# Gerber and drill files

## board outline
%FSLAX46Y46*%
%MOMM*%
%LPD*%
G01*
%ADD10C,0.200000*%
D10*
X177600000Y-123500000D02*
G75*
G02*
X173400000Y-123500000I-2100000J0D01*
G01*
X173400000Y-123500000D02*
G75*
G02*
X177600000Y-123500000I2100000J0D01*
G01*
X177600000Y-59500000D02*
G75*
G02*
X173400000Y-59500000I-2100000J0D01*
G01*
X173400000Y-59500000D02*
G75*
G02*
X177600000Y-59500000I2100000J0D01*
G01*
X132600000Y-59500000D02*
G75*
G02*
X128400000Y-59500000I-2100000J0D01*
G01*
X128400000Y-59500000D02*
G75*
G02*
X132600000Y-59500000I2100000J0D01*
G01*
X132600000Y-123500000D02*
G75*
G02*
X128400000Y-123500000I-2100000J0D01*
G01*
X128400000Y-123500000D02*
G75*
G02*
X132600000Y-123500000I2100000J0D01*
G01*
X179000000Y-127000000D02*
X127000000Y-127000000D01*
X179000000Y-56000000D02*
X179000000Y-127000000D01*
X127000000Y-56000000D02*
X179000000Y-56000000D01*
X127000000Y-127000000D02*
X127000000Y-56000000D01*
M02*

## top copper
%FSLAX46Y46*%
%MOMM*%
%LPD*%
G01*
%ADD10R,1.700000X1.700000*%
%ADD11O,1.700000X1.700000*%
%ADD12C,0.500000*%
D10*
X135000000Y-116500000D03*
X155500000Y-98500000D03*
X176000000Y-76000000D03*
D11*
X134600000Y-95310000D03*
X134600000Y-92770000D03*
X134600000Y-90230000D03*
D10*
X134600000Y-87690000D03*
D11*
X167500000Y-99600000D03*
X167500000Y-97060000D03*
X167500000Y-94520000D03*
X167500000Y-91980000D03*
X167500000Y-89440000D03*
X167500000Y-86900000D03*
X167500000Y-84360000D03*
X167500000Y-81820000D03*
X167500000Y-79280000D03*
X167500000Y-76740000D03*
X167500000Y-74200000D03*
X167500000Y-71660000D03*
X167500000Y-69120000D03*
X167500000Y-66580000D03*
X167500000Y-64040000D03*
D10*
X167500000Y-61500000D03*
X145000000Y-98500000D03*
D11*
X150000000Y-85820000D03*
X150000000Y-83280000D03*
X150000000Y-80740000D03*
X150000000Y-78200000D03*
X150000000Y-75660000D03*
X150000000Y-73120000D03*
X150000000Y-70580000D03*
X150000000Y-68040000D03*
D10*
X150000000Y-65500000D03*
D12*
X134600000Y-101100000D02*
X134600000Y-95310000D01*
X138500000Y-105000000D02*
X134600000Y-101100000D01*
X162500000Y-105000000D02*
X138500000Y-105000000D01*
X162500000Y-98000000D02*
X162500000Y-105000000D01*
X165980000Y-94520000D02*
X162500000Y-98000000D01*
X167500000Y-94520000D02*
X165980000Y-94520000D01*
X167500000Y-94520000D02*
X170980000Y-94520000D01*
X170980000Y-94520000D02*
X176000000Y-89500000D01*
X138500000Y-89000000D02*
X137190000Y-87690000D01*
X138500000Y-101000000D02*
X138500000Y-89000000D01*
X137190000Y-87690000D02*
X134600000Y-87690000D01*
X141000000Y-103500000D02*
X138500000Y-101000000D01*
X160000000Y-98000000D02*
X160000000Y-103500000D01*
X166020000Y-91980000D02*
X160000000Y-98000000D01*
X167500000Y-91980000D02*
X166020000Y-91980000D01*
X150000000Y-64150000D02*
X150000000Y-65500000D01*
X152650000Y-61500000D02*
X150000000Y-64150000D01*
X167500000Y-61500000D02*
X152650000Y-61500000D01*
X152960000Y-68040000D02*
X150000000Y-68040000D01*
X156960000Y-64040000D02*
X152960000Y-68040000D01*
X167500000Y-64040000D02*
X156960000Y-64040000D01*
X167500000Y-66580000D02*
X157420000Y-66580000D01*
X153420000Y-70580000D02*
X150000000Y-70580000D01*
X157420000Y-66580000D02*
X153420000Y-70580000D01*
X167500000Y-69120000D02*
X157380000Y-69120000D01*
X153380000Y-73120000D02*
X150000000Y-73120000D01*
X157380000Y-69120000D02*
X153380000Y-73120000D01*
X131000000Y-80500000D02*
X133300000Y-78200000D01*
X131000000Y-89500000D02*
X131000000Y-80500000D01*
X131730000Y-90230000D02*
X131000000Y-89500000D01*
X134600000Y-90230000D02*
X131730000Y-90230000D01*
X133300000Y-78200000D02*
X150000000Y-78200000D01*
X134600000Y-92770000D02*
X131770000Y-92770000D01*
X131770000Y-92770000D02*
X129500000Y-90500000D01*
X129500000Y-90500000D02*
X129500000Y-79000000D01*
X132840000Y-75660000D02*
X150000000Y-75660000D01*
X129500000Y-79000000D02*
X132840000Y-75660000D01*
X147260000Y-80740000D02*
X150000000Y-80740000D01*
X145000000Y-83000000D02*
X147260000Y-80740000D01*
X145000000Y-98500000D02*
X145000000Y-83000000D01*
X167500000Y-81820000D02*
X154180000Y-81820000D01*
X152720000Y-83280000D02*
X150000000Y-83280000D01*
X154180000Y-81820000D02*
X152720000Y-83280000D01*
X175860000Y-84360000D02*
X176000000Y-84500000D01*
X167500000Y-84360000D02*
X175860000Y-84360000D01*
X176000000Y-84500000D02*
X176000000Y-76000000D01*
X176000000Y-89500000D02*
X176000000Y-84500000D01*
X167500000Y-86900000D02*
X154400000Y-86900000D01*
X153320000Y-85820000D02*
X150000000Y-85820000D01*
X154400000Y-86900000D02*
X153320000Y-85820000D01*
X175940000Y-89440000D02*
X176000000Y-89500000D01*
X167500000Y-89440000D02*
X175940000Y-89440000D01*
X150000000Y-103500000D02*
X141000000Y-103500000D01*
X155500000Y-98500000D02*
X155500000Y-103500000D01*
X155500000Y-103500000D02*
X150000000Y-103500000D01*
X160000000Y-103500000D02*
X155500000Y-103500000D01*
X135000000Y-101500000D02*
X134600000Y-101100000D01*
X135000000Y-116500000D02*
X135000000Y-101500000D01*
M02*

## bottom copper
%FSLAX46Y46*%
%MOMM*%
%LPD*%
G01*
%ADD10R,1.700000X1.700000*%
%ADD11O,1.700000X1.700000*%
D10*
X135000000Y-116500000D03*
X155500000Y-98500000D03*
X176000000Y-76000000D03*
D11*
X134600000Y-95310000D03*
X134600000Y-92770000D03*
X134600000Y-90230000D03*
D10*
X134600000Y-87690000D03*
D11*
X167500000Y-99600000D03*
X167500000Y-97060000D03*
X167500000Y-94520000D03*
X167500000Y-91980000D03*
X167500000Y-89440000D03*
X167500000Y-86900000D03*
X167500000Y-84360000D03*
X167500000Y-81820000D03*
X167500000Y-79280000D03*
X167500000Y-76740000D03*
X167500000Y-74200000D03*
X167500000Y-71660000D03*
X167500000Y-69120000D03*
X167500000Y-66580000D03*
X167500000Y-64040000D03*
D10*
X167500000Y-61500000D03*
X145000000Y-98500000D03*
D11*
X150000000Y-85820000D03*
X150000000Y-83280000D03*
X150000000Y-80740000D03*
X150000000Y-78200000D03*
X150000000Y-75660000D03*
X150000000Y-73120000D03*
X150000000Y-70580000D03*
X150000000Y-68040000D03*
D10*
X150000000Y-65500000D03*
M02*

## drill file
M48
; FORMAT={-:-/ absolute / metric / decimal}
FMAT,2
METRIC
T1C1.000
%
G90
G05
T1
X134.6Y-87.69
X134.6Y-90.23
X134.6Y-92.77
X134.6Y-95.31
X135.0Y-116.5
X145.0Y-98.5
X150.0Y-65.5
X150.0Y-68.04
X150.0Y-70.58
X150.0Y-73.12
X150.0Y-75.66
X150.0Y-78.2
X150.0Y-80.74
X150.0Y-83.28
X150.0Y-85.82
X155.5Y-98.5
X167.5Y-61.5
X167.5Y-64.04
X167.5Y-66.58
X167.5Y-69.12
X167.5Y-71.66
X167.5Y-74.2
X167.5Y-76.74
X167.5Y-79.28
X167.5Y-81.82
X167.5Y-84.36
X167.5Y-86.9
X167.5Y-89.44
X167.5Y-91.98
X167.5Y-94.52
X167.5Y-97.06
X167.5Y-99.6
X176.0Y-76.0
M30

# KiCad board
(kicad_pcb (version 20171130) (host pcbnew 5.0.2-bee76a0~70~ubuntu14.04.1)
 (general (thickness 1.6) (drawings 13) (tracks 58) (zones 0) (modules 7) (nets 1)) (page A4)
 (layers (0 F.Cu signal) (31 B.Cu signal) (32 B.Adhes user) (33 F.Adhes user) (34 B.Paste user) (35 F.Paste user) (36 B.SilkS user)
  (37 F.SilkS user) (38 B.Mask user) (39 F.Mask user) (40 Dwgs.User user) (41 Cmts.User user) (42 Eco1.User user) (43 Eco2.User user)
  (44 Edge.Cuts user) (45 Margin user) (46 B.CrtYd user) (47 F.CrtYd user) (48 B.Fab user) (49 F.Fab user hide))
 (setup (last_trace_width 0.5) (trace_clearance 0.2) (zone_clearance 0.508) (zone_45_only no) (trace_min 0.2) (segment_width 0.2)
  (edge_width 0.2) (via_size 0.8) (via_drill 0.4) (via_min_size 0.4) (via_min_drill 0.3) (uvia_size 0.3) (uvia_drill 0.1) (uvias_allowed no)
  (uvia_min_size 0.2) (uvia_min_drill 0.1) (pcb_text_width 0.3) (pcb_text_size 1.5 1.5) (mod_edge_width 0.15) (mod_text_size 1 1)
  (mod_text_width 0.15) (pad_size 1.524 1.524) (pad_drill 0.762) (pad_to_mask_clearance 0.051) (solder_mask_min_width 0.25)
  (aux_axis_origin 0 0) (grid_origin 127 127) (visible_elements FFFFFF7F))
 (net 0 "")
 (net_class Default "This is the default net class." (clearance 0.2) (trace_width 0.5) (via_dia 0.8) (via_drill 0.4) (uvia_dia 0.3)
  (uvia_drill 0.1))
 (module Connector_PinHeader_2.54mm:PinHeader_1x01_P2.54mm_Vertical (layer F.Cu) (at 135 116.5)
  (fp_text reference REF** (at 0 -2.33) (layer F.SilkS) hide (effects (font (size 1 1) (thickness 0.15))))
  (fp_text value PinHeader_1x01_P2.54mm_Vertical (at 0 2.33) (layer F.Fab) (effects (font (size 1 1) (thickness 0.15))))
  (pad 1 thru_hole rect (at 0 0) (size 1.7 1.7) (drill 1) (layers *.Cu *.Mask)))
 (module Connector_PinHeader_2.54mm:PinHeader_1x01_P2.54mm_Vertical (layer F.Cu) (at 155.5 98.5)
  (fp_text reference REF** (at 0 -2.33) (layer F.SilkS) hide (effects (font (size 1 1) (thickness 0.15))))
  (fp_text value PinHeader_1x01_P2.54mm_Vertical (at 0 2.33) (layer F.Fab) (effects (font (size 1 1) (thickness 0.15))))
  (pad 1 thru_hole rect (at 0 0) (size 1.7 1.7) (drill 1) (layers *.Cu *.Mask)))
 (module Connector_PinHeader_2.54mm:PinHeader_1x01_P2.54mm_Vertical (layer F.Cu) (at 176 76)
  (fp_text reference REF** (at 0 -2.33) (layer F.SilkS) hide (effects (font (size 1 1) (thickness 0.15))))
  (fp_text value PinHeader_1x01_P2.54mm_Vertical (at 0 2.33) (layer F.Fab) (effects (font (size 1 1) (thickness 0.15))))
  (pad 1 thru_hole rect (at 0 0) (size 1.7 1.7) (drill 1) (layers *.Cu *.Mask)))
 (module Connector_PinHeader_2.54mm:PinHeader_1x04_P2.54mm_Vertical (layer F.Cu) (at 134.6 87.69)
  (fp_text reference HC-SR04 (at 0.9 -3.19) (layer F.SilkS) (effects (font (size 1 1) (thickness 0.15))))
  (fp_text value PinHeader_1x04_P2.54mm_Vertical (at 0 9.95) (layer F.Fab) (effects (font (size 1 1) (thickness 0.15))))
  (pad 4 thru_hole oval (at 0 7.62) (size 1.7 1.7) (drill 1) (layers *.Cu *.Mask))
  (pad 3 thru_hole oval (at 0 5.08) (size 1.7 1.7) (drill 1) (layers *.Cu *.Mask))
  (pad 2 thru_hole oval (at 0 2.54) (size 1.7 1.7) (drill 1) (layers *.Cu *.Mask))
  (pad 1 thru_hole rect (at 0 0) (size 1.7 1.7) (drill 1) (layers *.Cu *.Mask)))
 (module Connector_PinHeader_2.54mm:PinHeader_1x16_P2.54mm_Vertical (layer F.Cu) (at 167.5 61.5)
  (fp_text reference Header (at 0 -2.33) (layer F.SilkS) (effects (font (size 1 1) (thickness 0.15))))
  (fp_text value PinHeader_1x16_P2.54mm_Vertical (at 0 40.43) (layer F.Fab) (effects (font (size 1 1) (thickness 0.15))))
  (pad 16 thru_hole oval (at 0 38.1) (size 1.7 1.7) (drill 1) (layers *.Cu *.Mask))
  (pad 15 thru_hole oval (at 0 35.56) (size 1.7 1.7) (drill 1) (layers *.Cu *.Mask))
  (pad 14 thru_hole oval (at 0 33.02) (size 1.7 1.7) (drill 1) (layers *.Cu *.Mask))
  (pad 13 thru_hole oval (at 0 30.48) (size 1.7 1.7) (drill 1) (layers *.Cu *.Mask))
  (pad 12 thru_hole oval (at 0 27.94) (size 1.7 1.7) (drill 1) (layers *.Cu *.Mask))
  (pad 11 thru_hole oval (at 0 25.4) (size 1.7 1.7) (drill 1) (layers *.Cu *.Mask))
  (pad 10 thru_hole oval (at 0 22.86) (size 1.7 1.7) (drill 1) (layers *.Cu *.Mask))
  (pad 9 thru_hole oval (at 0 20.32) (size 1.7 1.7) (drill 1) (layers *.Cu *.Mask))
  (pad 8 thru_hole oval (at 0 17.78) (size 1.7 1.7) (drill 1) (layers *.Cu *.Mask))
  (pad 7 thru_hole oval (at 0 15.24) (size 1.7 1.7) (drill 1) (layers *.Cu *.Mask))
  (pad 6 thru_hole oval (at 0 12.7) (size 1.7 1.7) (drill 1) (layers *.Cu *.Mask))
  (pad 5 thru_hole oval (at 0 10.16) (size 1.7 1.7) (drill 1) (layers *.Cu *.Mask))
  (pad 4 thru_hole oval (at 0 7.62) (size 1.7 1.7) (drill 1) (layers *.Cu *.Mask))
  (pad 3 thru_hole oval (at 0 5.08) (size 1.7 1.7) (drill 1) (layers *.Cu *.Mask))
  (pad 2 thru_hole oval (at 0 2.54) (size 1.7 1.7) (drill 1) (layers *.Cu *.Mask))
  (pad 1 thru_hole rect (at 0 0) (size 1.7 1.7) (drill 1) (layers *.Cu *.Mask)))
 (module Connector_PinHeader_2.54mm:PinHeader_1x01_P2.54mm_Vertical (layer F.Cu) (at 145 98.5)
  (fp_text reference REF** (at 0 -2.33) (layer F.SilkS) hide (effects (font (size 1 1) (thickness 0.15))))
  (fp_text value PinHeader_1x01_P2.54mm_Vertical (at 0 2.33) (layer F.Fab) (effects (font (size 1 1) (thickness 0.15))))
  (pad 1 thru_hole rect (at 0 0) (size 1.7 1.7) (drill 1) (layers *.Cu *.Mask)))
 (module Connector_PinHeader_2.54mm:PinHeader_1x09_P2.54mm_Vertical (layer F.Cu) (at 150 65.5)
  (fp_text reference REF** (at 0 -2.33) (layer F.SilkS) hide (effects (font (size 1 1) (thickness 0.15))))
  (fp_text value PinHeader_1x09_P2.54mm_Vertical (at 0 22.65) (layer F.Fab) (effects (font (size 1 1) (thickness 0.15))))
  (pad 9 thru_hole oval (at 0 20.32) (size 1.7 1.7) (drill 1) (layers *.Cu *.Mask))
  (pad 8 thru_hole oval (at 0 17.78) (size 1.7 1.7) (drill 1) (layers *.Cu *.Mask))
  (pad 7 thru_hole oval (at 0 15.24) (size 1.7 1.7) (drill 1) (layers *.Cu *.Mask))
  (pad 6 thru_hole oval (at 0 12.7) (size 1.7 1.7) (drill 1) (layers *.Cu *.Mask))
  (pad 5 thru_hole oval (at 0 10.16) (size 1.7 1.7) (drill 1) (layers *.Cu *.Mask))
  (pad 4 thru_hole oval (at 0 7.62) (size 1.7 1.7) (drill 1) (layers *.Cu *.Mask))
  (pad 3 thru_hole oval (at 0 5.08) (size 1.7 1.7) (drill 1) (layers *.Cu *.Mask))
  (pad 2 thru_hole oval (at 0 2.54) (size 1.7 1.7) (drill 1) (layers *.Cu *.Mask))
  (pad 1 thru_hole rect (at 0 0) (size 1.7 1.7) (drill 1) (layers *.Cu *.Mask)))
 (gr_circle (center 175.5 123.5) (end 177.6 123.5) (layer Edge.Cuts) (width 0.2))
 (gr_circle (center 175.5 59.5) (end 177.6 59.5) (layer Edge.Cuts) (width 0.2))
 (gr_circle (center 130.5 59.5) (end 132.6 59.5) (layer Edge.Cuts) (width 0.2))
 (gr_circle (center 130.5 123.5) (end 132.6 123.5) (layer Edge.Cuts) (width 0.2))
 (gr_line (start 179 127) (end 127 127) (layer Edge.Cuts) (width 0.2))
 (gr_line (start 179 56) (end 179 127) (layer Edge.Cuts) (width 0.2))
 (gr_line (start 127 56) (end 179 56) (layer Edge.Cuts) (width 0.2))
 (gr_line (start 127 127) (end 127 56) (layer Edge.Cuts) (width 0.2))
 (segment (start 134.6 101.1) (end 134.6 95.31) (width 0.5) (layer F.Cu) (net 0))
 (segment (start 138.5 105) (end 134.6 101.1) (width 0.5) (layer F.Cu) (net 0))
 (segment (start 162.5 105) (end 138.5 105) (width 0.5) (layer F.Cu) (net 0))
 (segment (start 162.5 98) (end 162.5 105) (width 0.5) (layer F.Cu) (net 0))
 (segment (start 165.98 94.52) (end 162.5 98) (width 0.5) (layer F.Cu) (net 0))
 (segment (start 167.5 94.52) (end 165.98 94.52) (width 0.5) (layer F.Cu) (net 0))
 (segment (start 167.5 94.52) (end 170.98 94.52) (width 0.5) (layer F.Cu) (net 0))
 (segment (start 170.98 94.52) (end 176 89.5) (width 0.5) (layer F.Cu) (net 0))
 (segment (start 138.5 89) (end 137.19 87.69) (width 0.5) (layer F.Cu) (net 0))
 (segment (start 138.5 101) (end 138.5 89) (width 0.5) (layer F.Cu) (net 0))
 (segment (start 137.19 87.69) (end 134.6 87.69) (width 0.5) (layer F.Cu) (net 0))
 (segment (start 141 103.5) (end 138.5 101) (width 0.5) (layer F.Cu) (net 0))
 (segment (start 160 98) (end 160 103.5) (width 0.5) (layer F.Cu) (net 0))
 (segment (start 166.02 91.98) (end 160 98) (width 0.5) (layer F.Cu) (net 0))
 (segment (start 167.5 91.98) (end 166.02 91.98) (width 0.5) (layer F.Cu) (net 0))
 (segment (start 150 64.15) (end 150 65.5) (width 0.5) (layer F.Cu) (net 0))
 (segment (start 152.65 61.5) (end 150 64.15) (width 0.5) (layer F.Cu) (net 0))
 (segment (start 167.5 61.5) (end 152.65 61.5) (width 0.5) (layer F.Cu) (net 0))
 (segment (start 152.96 68.04) (end 150 68.04) (width 0.5) (layer F.Cu) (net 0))
 (segment (start 156.96 64.04) (end 152.96 68.04) (width 0.5) (layer F.Cu) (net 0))
 (segment (start 167.5 64.04) (end 156.96 64.04) (width 0.5) (layer F.Cu) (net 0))
 (segment (start 167.5 66.58) (end 157.42 66.58) (width 0.5) (layer F.Cu) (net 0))
 (segment (start 153.42 70.58) (end 150 70.58) (width 0.5) (layer F.Cu) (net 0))
 (segment (start 157.42 66.58) (end 153.42 70.58) (width 0.5) (layer F.Cu) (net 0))
 (segment (start 167.5 69.12) (end 157.38 69.12) (width 0.5) (layer F.Cu) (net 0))
 (segment (start 153.38 73.12) (end 150 73.12) (width 0.5) (layer F.Cu) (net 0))
 (segment (start 157.38 69.12) (end 153.38 73.12) (width 0.5) (layer F.Cu) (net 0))
 (segment (start 131 80.5) (end 133.3 78.2) (width 0.5) (layer F.Cu) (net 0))
 (segment (start 131 89.5) (end 131 80.5) (width 0.5) (layer F.Cu) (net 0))
 (segment (start 131.73 90.23) (end 131 89.5) (width 0.5) (layer F.Cu) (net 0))
 (segment (start 134.6 90.23) (end 131.73 90.23) (width 0.5) (layer F.Cu) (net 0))
 (segment (start 133.3 78.2) (end 150 78.2) (width 0.5) (layer F.Cu) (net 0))
 (segment (start 134.6 92.77) (end 131.77 92.77) (width 0.5) (layer F.Cu) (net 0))
 (segment (start 131.77 92.77) (end 129.5 90.5) (width 0.5) (layer F.Cu) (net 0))
 (segment (start 129.5 90.5) (end 129.5 79) (width 0.5) (layer F.Cu) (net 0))
 (segment (start 132.84 75.66) (end 150 75.66) (width 0.5) (layer F.Cu) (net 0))
 (segment (start 129.5 79) (end 132.84 75.66) (width 0.5) (layer F.Cu) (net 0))
 (segment (start 147.26 80.74) (end 150 80.74) (width 0.5) (layer F.Cu) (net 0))
 (segment (start 145 83) (end 147.26 80.74) (width 0.5) (layer F.Cu) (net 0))
 (segment (start 145 98.5) (end 145 83) (width 0.5) (layer F.Cu) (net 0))
 (segment (start 167.5 81.82) (end 154.18 81.82) (width 0.5) (layer F.Cu) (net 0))
 (segment (start 152.72 83.28) (end 150 83.28) (width 0.5) (layer F.Cu) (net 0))
 (segment (start 154.18 81.82) (end 152.72 83.28) (width 0.5) (layer F.Cu) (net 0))
 (segment (start 175.86 84.36) (end 176 84.5) (width 0.5) (layer F.Cu) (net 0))
 (segment (start 167.5 84.36) (end 175.86 84.36) (width 0.5) (layer F.Cu) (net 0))
 (segment (start 176 84.5) (end 176 76) (width 0.5) (layer F.Cu) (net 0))
 (segment (start 176 89.5) (end 176 84.5) (width 0.5) (layer F.Cu) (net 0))
 (segment (start 167.5 86.9) (end 154.4 86.9) (width 0.5) (layer F.Cu) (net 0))
 (segment (start 153.32 85.82) (end 150 85.82) (width 0.5) (layer F.Cu) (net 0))
 (segment (start 154.4 86.9) (end 153.32 85.82) (width 0.5) (layer F.Cu) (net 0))
 (segment (start 175.94 89.44) (end 176 89.5) (width 0.5) (layer F.Cu) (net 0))
 (segment (start 167.5 89.44) (end 175.94 89.44) (width 0.5) (layer F.Cu) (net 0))
 (segment (start 150 103.5) (end 141 103.5) (width 0.5) (layer F.Cu) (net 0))
 (segment (start 155.5 98.5) (end 155.5 103.5) (width 0.5) (layer F.Cu) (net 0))
 (segment (start 155.5 103.5) (end 150 103.5) (width 0.5) (layer F.Cu) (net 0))
 (segment (start 160 103.5) (end 155.5 103.5) (width 0.5) (layer F.Cu) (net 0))
 (segment (start 135 101.5) (end 134.6 101.1) (width 0.5) (layer F.Cu) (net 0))
 (segment (start 135 116.5) (end 135 101.5) (width 0.5) (layer F.Cu) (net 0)))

